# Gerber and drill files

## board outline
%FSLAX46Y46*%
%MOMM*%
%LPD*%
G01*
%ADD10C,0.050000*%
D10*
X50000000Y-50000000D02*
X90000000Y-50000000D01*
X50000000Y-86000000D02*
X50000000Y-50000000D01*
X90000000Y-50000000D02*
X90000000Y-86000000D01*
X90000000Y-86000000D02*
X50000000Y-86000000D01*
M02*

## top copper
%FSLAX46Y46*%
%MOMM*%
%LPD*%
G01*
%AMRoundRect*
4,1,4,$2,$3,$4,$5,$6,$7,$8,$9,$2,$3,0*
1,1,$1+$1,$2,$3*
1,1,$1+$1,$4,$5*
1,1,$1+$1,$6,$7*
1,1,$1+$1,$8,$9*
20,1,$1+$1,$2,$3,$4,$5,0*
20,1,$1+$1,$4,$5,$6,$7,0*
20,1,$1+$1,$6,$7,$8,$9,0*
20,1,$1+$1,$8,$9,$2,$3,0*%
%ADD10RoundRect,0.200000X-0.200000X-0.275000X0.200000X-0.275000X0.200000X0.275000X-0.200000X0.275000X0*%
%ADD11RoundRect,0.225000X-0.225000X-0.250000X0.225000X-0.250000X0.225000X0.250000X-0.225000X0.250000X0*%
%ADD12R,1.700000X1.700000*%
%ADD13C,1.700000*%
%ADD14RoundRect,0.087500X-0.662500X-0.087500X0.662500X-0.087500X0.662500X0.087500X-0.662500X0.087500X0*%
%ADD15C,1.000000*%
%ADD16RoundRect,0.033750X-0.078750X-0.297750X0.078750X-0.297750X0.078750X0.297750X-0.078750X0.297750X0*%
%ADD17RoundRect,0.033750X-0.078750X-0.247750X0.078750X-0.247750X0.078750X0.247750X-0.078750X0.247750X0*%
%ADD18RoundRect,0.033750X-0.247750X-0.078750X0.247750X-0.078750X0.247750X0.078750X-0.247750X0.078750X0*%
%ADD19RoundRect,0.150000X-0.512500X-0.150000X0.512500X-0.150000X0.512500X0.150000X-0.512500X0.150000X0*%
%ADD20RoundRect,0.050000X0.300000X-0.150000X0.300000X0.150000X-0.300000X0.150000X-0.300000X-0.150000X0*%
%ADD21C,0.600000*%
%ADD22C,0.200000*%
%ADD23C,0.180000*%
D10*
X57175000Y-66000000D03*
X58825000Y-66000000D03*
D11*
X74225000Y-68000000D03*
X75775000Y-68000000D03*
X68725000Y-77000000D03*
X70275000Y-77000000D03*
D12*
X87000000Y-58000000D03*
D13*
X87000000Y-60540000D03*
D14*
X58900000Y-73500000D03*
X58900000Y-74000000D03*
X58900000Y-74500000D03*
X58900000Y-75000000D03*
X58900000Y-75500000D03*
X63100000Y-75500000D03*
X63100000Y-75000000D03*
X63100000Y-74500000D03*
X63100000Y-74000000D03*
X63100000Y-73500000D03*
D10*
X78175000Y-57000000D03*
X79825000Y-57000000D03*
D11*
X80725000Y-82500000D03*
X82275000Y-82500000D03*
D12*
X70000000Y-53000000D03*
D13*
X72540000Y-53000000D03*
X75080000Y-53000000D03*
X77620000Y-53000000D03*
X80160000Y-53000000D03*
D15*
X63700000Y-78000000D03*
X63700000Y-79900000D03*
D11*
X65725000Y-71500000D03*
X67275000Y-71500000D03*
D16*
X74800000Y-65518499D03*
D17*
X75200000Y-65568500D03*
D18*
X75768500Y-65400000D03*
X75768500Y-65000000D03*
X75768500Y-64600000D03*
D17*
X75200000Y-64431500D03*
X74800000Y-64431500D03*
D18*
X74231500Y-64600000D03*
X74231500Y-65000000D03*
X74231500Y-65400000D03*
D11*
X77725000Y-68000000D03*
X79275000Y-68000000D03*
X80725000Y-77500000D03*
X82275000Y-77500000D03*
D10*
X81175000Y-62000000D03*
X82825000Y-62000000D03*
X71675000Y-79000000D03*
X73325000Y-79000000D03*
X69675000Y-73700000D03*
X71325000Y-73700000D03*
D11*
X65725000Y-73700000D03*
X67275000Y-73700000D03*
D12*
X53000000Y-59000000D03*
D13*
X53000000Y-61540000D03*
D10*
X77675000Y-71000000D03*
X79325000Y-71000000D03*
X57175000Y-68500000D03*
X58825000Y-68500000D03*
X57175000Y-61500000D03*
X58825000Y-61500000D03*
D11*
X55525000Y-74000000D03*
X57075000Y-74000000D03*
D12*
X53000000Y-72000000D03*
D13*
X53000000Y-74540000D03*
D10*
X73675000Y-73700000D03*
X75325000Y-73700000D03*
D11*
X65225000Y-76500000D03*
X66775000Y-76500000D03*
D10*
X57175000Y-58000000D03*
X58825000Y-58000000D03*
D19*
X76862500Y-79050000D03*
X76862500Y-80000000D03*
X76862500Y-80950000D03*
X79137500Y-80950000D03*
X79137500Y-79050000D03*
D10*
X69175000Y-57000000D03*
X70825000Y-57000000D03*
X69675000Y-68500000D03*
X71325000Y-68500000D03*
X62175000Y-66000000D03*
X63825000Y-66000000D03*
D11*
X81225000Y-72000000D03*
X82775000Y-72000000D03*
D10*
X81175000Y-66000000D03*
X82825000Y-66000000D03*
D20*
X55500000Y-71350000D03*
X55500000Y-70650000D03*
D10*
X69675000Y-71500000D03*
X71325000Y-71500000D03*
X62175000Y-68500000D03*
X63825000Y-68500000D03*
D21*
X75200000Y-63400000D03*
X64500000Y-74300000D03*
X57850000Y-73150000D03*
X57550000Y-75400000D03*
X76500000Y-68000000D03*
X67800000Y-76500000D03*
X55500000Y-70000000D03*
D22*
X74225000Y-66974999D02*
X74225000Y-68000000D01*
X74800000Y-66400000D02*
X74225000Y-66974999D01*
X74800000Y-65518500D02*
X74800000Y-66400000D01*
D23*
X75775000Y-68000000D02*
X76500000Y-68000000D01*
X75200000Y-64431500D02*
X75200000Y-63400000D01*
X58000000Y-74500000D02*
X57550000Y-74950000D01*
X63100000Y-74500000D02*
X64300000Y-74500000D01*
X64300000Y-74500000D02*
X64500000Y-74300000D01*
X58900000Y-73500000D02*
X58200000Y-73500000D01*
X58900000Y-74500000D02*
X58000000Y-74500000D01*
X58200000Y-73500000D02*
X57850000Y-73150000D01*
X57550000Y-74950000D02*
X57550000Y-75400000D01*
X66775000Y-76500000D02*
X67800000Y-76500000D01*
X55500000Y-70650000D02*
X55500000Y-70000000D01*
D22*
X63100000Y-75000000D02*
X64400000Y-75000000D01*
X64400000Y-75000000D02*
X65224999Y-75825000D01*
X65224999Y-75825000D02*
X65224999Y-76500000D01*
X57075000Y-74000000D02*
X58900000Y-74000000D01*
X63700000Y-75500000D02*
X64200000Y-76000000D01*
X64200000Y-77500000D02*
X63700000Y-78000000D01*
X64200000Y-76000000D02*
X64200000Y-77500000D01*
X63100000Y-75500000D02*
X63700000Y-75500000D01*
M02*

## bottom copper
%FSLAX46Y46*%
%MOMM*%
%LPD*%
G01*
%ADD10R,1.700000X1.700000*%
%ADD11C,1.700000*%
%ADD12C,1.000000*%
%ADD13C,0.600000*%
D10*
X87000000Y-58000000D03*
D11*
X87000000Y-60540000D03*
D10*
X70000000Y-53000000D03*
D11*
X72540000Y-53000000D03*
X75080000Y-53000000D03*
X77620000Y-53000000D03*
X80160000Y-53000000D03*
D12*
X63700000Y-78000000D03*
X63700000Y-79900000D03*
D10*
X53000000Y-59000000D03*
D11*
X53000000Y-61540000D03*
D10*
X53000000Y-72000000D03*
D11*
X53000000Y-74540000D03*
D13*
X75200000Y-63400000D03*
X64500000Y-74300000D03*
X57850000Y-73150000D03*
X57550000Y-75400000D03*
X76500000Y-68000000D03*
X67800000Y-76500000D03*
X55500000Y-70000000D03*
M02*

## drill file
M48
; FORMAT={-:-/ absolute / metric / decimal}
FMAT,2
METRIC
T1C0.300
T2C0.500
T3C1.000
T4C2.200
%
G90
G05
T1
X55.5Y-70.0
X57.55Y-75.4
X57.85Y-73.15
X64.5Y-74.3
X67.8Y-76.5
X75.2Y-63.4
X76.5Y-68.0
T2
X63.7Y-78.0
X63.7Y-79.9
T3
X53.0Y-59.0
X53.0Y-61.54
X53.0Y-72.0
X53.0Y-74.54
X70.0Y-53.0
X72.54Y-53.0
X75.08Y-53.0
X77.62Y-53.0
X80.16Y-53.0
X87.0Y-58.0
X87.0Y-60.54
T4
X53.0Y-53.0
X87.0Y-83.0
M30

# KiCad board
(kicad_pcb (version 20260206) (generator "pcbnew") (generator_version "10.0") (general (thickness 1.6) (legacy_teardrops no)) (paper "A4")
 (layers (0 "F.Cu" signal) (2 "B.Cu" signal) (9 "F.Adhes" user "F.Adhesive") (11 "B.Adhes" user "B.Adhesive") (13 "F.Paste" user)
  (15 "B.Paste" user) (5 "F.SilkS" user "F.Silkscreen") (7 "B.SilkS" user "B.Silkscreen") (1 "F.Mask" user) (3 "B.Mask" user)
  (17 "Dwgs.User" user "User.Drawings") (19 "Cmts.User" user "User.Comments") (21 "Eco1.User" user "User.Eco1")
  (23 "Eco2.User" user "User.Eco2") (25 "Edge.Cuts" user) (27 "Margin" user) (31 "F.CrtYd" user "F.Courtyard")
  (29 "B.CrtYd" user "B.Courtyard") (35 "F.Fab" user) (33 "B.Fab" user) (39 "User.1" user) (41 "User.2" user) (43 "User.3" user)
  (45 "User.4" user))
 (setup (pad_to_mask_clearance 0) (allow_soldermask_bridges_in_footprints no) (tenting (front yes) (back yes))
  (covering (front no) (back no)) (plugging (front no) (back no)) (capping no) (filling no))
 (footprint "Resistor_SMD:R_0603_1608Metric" (layer "F.Cu") (at 58 66)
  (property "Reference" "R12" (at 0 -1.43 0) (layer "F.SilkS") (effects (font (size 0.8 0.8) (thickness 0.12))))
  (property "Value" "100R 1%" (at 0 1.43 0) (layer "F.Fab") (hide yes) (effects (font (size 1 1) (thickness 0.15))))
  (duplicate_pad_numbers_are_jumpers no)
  (pad "1" smd roundrect (at -0.825 0) (size 0.8 0.95) (layers "F.Cu" "F.Mask" "F.Paste") (roundrect_rratio 0.25) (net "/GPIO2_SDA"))
  (pad "2" smd roundrect (at 0.825 0) (size 0.8 0.95) (layers "F.Cu" "F.Mask" "F.Paste") (roundrect_rratio 0.25) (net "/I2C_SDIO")))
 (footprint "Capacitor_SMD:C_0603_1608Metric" (layer "F.Cu") (at 75 68)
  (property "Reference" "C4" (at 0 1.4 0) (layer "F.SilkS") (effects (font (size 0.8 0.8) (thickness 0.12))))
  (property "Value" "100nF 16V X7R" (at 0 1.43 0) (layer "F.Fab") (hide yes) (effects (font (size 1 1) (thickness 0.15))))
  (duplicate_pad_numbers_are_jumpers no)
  (pad "1" smd roundrect (at -0.775 0) (size 0.9 0.95) (layers "F.Cu" "F.Mask" "F.Paste") (roundrect_rratio 0.25) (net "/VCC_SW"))
  (pad "2" smd roundrect (at 0.775 0) (size 0.9 0.95) (layers "F.Cu" "F.Mask" "F.Paste") (roundrect_rratio 0.25) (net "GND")))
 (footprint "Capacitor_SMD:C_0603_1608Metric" (layer "F.Cu") (at 69.5 77)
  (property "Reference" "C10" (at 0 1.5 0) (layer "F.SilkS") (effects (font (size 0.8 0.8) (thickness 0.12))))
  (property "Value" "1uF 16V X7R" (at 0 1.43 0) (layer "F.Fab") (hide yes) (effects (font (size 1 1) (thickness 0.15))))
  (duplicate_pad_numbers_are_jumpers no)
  (pad "1" smd roundrect (at -0.775 0) (size 0.9 0.95) (layers "F.Cu" "F.Mask" "F.Paste") (roundrect_rratio 0.25) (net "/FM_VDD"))
  (pad "2" smd roundrect (at 0.775 0) (size 0.9 0.95) (layers "F.Cu" "F.Mask" "F.Paste") (roundrect_rratio 0.25) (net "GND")))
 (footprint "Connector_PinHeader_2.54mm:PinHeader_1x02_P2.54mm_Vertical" (layer "F.Cu") (at 87 58)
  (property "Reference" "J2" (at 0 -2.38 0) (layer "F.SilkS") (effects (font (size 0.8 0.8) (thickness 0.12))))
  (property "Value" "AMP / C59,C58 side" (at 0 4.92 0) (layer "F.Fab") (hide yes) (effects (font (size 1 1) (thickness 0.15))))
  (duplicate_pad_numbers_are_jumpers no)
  (pad "1" thru_hole rect (at 0 0) (size 1.7 1.7) (drill 1) (layers "*.Cu" "*.Mask") (remove_unused_layers no) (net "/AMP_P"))
  (pad "2" thru_hole circle (at 0 2.54) (size 1.7 1.7) (drill 1) (layers "*.Cu" "*.Mask") (remove_unused_layers no) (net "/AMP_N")))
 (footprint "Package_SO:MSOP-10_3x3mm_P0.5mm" (layer "F.Cu") (at 61 74.5)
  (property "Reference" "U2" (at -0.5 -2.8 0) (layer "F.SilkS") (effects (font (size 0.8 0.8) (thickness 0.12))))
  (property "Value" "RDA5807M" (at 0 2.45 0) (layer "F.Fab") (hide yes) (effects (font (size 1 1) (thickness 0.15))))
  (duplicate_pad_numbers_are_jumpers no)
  (pad "1" smd roundrect (at -2.1 -1) (size 1.5 0.35) (layers "F.Cu" "F.Mask" "F.Paste") (roundrect_rratio 0.25) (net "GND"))
  (pad "2" smd roundrect (at -2.1 -0.5) (size 1.5 0.35) (layers "F.Cu" "F.Mask" "F.Paste") (roundrect_rratio 0.25) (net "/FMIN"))
  (pad "3" smd roundrect (at -2.1 0) (size 1.5 0.35) (layers "F.Cu" "F.Mask" "F.Paste") (roundrect_rratio 0.25) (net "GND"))
  (pad "4" smd roundrect (at -2.1 0.5) (size 1.5 0.35) (layers "F.Cu" "F.Mask" "F.Paste") (roundrect_rratio 0.25) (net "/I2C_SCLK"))
  (pad "5" smd roundrect (at -2.1 1) (size 1.5 0.35) (layers "F.Cu" "F.Mask" "F.Paste") (roundrect_rratio 0.25) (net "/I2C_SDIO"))
  (pad "6" smd roundrect (at 2.1 1) (size 1.5 0.35) (layers "F.Cu" "F.Mask" "F.Paste") (roundrect_rratio 0.25) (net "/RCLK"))
  (pad "7" smd roundrect (at 2.1 0.5) (size 1.5 0.35) (layers "F.Cu" "F.Mask" "F.Paste") (roundrect_rratio 0.25) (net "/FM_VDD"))
  (pad "8" smd roundrect (at 2.1 0) (size 1.5 0.35) (layers "F.Cu" "F.Mask" "F.Paste") (roundrect_rratio 0.25) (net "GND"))
  (pad "9" smd roundrect (at 2.1 -0.5) (size 1.5 0.35) (layers "F.Cu" "F.Mask" "F.Paste") (roundrect_rratio 0.25) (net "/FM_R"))
  (pad "10" smd roundrect (at 2.1 -1) (size 1.5 0.35) (layers "F.Cu" "F.Mask" "F.Paste") (roundrect_rratio 0.25) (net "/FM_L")))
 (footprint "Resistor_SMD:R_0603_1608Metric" (layer "F.Cu") (at 79 57)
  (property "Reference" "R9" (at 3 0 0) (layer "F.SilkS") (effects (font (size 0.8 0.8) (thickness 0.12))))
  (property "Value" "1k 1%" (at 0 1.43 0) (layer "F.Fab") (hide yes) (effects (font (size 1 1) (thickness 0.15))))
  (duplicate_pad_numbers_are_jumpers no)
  (pad "1" smd roundrect (at -0.825 0) (size 0.8 0.95) (layers "F.Cu" "F.Mask" "F.Paste") (roundrect_rratio 0.25) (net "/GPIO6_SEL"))
  (pad "2" smd roundrect (at 0.825 0) (size 0.8 0.95) (layers "F.Cu" "F.Mask" "F.Paste") (roundrect_rratio 0.25) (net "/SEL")))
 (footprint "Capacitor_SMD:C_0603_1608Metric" (layer "F.Cu") (at 81.5 82.5)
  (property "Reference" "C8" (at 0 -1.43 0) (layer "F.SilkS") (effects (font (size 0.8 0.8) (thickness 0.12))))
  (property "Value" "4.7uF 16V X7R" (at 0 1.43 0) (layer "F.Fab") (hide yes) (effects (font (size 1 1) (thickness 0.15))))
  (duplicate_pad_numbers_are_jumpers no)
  (pad "1" smd roundrect (at -0.775 0) (size 0.9 0.95) (layers "F.Cu" "F.Mask" "F.Paste") (roundrect_rratio 0.25) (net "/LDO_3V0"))
  (pad "2" smd roundrect (at 0.775 0) (size 0.9 0.95) (layers "F.Cu" "F.Mask" "F.Paste") (roundrect_rratio 0.25) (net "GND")))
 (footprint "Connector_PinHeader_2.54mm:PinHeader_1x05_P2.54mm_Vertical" (layer "F.Cu") (at 70 53 90)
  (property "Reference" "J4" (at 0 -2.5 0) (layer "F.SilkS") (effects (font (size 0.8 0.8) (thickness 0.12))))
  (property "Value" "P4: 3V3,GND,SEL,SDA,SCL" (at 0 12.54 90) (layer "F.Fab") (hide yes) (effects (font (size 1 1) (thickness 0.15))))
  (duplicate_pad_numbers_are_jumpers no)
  (pad "1" thru_hole rect (at 0 0 90) (size 1.7 1.7) (drill 1) (layers "*.Cu" "*.Mask") (remove_unused_layers no) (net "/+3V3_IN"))
  (pad "2" thru_hole circle (at 0 2.54 90) (size 1.7 1.7) (drill 1) (layers "*.Cu" "*.Mask") (remove_unused_layers no) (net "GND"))
  (pad "3" thru_hole circle (at 0 5.08 90) (size 1.7 1.7) (drill 1) (layers "*.Cu" "*.Mask") (remove_unused_layers no) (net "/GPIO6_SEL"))
  (pad "4" thru_hole circle (at 0 7.62 90) (size 1.7 1.7) (drill 1) (layers "*.Cu" "*.Mask") (remove_unused_layers no) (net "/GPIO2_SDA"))
  (pad "5" thru_hole circle (at 0 10.16 90) (size 1.7 1.7) (drill 1) (layers "*.Cu" "*.Mask") (remove_unused_layers no) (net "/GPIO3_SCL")))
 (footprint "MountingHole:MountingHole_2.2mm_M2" (layer "F.Cu") (at 53 53)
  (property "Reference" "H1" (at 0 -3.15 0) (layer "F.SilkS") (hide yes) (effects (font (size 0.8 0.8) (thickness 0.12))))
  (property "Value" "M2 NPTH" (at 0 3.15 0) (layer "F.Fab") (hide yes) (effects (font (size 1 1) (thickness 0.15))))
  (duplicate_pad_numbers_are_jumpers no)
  (pad "" np_thru_hole circle (at 0 0) (size 2.2 2.2) (drill 2.2) (layers "*.Cu" "*.Mask")))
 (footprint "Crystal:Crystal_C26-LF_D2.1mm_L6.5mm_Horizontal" (layer "F.Cu") (at 63.7 78 -90)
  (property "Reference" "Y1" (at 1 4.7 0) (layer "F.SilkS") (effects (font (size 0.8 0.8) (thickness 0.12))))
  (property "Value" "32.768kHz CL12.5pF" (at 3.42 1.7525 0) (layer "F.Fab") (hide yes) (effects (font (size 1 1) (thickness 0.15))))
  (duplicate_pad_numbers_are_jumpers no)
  (pad "1" thru_hole circle (at 0 0 270) (size 1 1) (drill 0.5) (layers "*.Cu" "*.Mask") (remove_unused_layers no) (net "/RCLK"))
  (pad "2" thru_hole circle (at 1.9 0 270) (size 1 1) (drill 0.5) (layers "*.Cu" "*.Mask") (remove_unused_layers no) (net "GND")))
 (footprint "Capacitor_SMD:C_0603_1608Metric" (layer "F.Cu") (at 66.5 71.5)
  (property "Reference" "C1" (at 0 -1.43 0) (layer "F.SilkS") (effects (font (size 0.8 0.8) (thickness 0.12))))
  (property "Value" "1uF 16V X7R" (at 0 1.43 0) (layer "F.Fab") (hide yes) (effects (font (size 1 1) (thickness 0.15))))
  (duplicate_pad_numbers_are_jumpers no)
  (pad "1" smd roundrect (at -0.775 0) (size 0.9 0.95) (layers "F.Cu" "F.Mask" "F.Paste") (roundrect_rratio 0.25) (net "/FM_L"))
  (pad "2" smd roundrect (at 0.775 0) (size 0.9 0.95) (layers "F.Cu" "F.Mask" "F.Paste") (roundrect_rratio 0.25) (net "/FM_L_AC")))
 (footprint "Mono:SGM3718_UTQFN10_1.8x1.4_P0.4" (layer "F.Cu") (at 75 65)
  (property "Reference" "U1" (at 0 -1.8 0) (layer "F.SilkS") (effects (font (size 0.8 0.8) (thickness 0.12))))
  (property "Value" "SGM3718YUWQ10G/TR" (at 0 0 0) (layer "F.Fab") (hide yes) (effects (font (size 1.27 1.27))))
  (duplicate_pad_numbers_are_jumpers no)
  (pad "1" smd roundrect (at -0.2 0.518499) (size 0.225 0.663) (layers "F.Cu" "F.Mask" "F.Paste") (roundrect_rratio 0.15) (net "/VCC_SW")
   (thermal_bridge_angle 45))
  (pad "2" smd roundrect (at 0.2 0.5685) (size 0.225 0.563) (layers "F.Cu" "F.Mask" "F.Paste") (roundrect_rratio 0.15) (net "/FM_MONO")
   (thermal_bridge_angle 45))
  (pad "3" smd roundrect (at 0.7685 0.4) (size 0.563 0.225) (layers "F.Cu" "F.Mask" "F.Paste") (roundrect_rratio 0.15) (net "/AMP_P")
   (thermal_bridge_angle 45))
  (pad "4" smd roundrect (at 0.7685 0) (size 0.563 0.225) (layers "F.Cu" "F.Mask" "F.Paste") (roundrect_rratio 0.15) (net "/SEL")
   (thermal_bridge_angle 45))
  (pad "5" smd roundrect (at 0.7685 -0.4) (size 0.563 0.225) (layers "F.Cu" "F.Mask" "F.Paste") (roundrect_rratio 0.15) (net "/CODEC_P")
   (thermal_bridge_angle 45))
  (pad "6" smd roundrect (at 0.2 -0.5685) (size 0.225 0.563) (layers "F.Cu" "F.Mask" "F.Paste") (roundrect_rratio 0.15) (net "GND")
   (thermal_bridge_angle 45))
  (pad "7" smd roundrect (at -0.2 -0.5685) (size 0.225 0.563) (layers "F.Cu" "F.Mask" "F.Paste") (roundrect_rratio 0.15) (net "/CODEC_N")
   (thermal_bridge_angle 45))
  (pad "8" smd roundrect (at -0.7685 -0.4) (size 0.563 0.225) (layers "F.Cu" "F.Mask" "F.Paste") (roundrect_rratio 0.15) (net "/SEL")
   (thermal_bridge_angle 45))
  (pad "9" smd roundrect (at -0.7685 0) (size 0.563 0.225) (layers "F.Cu" "F.Mask" "F.Paste") (roundrect_rratio 0.15) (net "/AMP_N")
   (thermal_bridge_angle 45))
  (pad "10" smd roundrect (at -0.7685 0.4) (size 0.563 0.225) (layers "F.Cu" "F.Mask" "F.Paste") (roundrect_rratio 0.15) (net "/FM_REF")
   (thermal_bridge_angle 45)))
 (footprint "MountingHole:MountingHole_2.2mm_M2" (layer "F.Cu") (at 87 83)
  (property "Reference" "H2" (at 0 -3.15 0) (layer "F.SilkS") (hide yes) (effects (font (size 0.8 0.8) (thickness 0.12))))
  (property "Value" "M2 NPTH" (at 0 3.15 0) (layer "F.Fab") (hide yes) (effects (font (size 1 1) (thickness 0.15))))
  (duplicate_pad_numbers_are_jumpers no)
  (pad "" np_thru_hole circle (at 0 0) (size 2.2 2.2) (drill 2.2) (layers "*.Cu" "*.Mask")))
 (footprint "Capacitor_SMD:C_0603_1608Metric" (layer "F.Cu") (at 78.5 68)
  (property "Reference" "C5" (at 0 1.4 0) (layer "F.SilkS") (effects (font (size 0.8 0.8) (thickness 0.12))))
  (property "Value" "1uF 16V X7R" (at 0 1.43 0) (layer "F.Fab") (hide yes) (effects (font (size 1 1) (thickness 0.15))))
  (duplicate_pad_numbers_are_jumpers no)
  (pad "1" smd roundrect (at -0.775 0) (size 0.9 0.95) (layers "F.Cu" "F.Mask" "F.Paste") (roundrect_rratio 0.25) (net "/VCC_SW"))
  (pad "2" smd roundrect (at 0.775 0) (size 0.9 0.95) (layers "F.Cu" "F.Mask" "F.Paste") (roundrect_rratio 0.25) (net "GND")))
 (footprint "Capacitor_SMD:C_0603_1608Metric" (layer "F.Cu") (at 81.5 77.5)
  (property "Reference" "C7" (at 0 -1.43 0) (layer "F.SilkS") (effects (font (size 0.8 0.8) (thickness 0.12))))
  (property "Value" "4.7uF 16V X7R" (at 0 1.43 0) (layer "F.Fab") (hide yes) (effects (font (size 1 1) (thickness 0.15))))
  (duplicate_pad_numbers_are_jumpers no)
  (pad "1" smd roundrect (at -0.775 0) (size 0.9 0.95) (layers "F.Cu" "F.Mask" "F.Paste") (roundrect_rratio 0.25) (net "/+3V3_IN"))
  (pad "2" smd roundrect (at 0.775 0) (size 0.9 0.95) (layers "F.Cu" "F.Mask" "F.Paste") (roundrect_rratio 0.25) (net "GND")))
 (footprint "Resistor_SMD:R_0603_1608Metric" (layer "F.Cu") (at 82 62)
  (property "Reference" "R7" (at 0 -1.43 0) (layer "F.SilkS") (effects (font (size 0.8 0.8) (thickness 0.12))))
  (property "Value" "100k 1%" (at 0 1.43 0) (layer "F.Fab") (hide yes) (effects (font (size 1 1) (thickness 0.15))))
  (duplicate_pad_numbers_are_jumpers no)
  (pad "1" smd roundrect (at -0.825 0) (size 0.8 0.95) (layers "F.Cu" "F.Mask" "F.Paste") (roundrect_rratio 0.25) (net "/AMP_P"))
  (pad "2" smd roundrect (at 0.825 0) (size 0.8 0.95) (layers "F.Cu" "F.Mask" "F.Paste") (roundrect_rratio 0.25) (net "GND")))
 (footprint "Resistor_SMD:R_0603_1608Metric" (layer "F.Cu") (at 72.5 79)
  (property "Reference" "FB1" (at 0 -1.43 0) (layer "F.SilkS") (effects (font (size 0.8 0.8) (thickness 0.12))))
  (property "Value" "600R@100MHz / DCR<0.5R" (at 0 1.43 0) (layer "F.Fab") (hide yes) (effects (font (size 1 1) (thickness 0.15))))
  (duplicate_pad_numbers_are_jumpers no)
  (pad "1" smd roundrect (at -0.825 0) (size 0.8 0.95) (layers "F.Cu" "F.Mask" "F.Paste") (roundrect_rratio 0.25) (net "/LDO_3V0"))
  (pad "2" smd roundrect (at 0.825 0) (size 0.8 0.95) (layers "F.Cu" "F.Mask" "F.Paste") (roundrect_rratio 0.25) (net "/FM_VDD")))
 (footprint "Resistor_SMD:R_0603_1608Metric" (layer "F.Cu") (at 70.5 73.7)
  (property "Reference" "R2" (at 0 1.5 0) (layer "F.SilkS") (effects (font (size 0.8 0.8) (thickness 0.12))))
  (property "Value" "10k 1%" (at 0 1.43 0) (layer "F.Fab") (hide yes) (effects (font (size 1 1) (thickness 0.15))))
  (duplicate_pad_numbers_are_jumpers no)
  (pad "1" smd roundrect (at -0.825 0) (size 0.8 0.95) (layers "F.Cu" "F.Mask" "F.Paste") (roundrect_rratio 0.25) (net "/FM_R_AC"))
  (pad "2" smd roundrect (at 0.825 0) (size 0.8 0.95) (layers "F.Cu" "F.Mask" "F.Paste") (roundrect_rratio 0.25) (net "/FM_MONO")))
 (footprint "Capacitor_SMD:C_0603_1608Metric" (layer "F.Cu") (at 66.5 73.7)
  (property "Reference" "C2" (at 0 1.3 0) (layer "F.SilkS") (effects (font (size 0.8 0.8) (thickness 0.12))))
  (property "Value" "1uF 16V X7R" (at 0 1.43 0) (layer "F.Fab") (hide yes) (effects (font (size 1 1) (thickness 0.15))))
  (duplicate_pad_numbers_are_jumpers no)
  (pad "1" smd roundrect (at -0.775 0) (size 0.9 0.95) (layers "F.Cu" "F.Mask" "F.Paste") (roundrect_rratio 0.25) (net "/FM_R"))
  (pad "2" smd roundrect (at 0.775 0) (size 0.9 0.95) (layers "F.Cu" "F.Mask" "F.Paste") (roundrect_rratio 0.25) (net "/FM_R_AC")))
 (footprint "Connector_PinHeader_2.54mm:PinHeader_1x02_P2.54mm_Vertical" (layer "F.Cu") (at 53 59)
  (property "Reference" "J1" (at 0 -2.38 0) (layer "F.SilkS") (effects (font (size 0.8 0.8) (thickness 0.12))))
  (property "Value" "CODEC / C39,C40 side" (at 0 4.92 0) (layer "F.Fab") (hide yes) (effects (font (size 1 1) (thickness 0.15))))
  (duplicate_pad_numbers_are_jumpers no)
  (pad "1" thru_hole rect (at 0 0) (size 1.7 1.7) (drill 1) (layers "*.Cu" "*.Mask") (remove_unused_layers no) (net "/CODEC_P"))
  (pad "2" thru_hole circle (at 0 2.54) (size 1.7 1.7) (drill 1) (layers "*.Cu" "*.Mask") (remove_unused_layers no) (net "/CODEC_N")))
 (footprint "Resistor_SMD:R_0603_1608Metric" (layer "F.Cu") (at 78.5 71)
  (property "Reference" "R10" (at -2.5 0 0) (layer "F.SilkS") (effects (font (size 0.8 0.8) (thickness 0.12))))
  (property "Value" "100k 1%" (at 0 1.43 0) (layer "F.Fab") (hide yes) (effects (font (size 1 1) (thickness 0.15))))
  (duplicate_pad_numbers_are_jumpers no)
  (pad "1" smd roundrect (at -0.825 0) (size 0.8 0.95) (layers "F.Cu" "F.Mask" "F.Paste") (roundrect_rratio 0.25) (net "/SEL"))
  (pad "2" smd roundrect (at 0.825 0) (size 0.8 0.95) (layers "F.Cu" "F.Mask" "F.Paste") (roundrect_rratio 0.25) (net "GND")))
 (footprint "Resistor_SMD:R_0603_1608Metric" (layer "F.Cu") (at 58 68.5)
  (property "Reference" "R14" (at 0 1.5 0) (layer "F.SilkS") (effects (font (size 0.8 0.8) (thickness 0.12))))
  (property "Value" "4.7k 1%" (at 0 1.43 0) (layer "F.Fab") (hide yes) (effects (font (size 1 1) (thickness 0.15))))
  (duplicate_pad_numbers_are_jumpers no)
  (pad "1" smd roundrect (at -0.825 0) (size 0.8 0.95) (layers "F.Cu" "F.Mask" "F.Paste") (roundrect_rratio 0.25) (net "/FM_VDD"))
  (pad "2" smd roundrect (at 0.825 0) (size 0.8 0.95) (layers "F.Cu" "F.Mask" "F.Paste") (roundrect_rratio 0.25) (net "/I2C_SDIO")))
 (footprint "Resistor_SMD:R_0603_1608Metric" (layer "F.Cu") (at 58 61.5)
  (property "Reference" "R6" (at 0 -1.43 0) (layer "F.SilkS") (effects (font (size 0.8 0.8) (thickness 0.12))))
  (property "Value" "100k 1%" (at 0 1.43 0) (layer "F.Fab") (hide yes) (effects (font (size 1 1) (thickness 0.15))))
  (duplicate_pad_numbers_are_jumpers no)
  (pad "1" smd roundrect (at -0.825 0) (size 0.8 0.95) (layers "F.Cu" "F.Mask" "F.Paste") (roundrect_rratio 0.25) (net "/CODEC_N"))
  (pad "2" smd roundrect (at 0.825 0) (size 0.8 0.95) (layers "F.Cu" "F.Mask" "F.Paste") (roundrect_rratio 0.25) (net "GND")))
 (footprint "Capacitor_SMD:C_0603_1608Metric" (layer "F.Cu") (at 56.3 74)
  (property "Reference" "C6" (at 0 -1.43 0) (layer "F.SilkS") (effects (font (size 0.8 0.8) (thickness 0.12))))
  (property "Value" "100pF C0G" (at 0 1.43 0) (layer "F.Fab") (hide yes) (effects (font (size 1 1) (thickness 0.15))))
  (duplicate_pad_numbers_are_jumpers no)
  (pad "1" smd roundrect (at -0.775 0) (size 0.9 0.95) (layers "F.Cu" "F.Mask" "F.Paste") (roundrect_rratio 0.25) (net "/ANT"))
  (pad "2" smd roundrect (at 0.775 0) (size 0.9 0.95) (layers "F.Cu" "F.Mask" "F.Paste") (roundrect_rratio 0.25) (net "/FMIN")))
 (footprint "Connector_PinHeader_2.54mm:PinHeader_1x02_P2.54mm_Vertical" (layer "F.Cu") (at 53 72)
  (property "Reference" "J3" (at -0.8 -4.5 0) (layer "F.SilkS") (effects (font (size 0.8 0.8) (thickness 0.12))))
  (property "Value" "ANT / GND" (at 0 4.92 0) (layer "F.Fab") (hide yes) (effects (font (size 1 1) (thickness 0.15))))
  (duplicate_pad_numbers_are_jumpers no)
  (pad "1" thru_hole rect (at 0 0) (size 1.7 1.7) (drill 1) (layers "*.Cu" "*.Mask") (remove_unused_layers no) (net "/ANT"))
  (pad "2" thru_hole circle (at 0 2.54) (size 1.7 1.7) (drill 1) (layers "*.Cu" "*.Mask") (remove_unused_layers no) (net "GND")))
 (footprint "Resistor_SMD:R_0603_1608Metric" (layer "F.Cu") (at 74.5 73.7)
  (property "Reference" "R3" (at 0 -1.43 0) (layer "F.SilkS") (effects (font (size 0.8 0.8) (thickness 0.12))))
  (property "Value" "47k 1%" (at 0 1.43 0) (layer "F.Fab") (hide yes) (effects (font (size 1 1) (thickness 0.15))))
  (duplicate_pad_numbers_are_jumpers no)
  (pad "1" smd roundrect (at -0.825 0) (size 0.8 0.95) (layers "F.Cu" "F.Mask" "F.Paste") (roundrect_rratio 0.25) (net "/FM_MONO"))
  (pad "2" smd roundrect (at 0.825 0) (size 0.8 0.95) (layers "F.Cu" "F.Mask" "F.Paste") (roundrect_rratio 0.25) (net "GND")))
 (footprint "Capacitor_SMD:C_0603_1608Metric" (layer "F.Cu") (at 66 76.5)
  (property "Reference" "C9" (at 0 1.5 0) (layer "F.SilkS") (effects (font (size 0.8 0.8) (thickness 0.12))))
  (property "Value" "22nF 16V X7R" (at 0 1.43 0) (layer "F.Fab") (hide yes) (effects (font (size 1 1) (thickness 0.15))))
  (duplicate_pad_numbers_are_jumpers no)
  (pad "1" smd roundrect (at -0.775 0) (size 0.9 0.95) (layers "F.Cu" "F.Mask" "F.Paste") (roundrect_rratio 0.25) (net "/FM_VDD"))
  (pad "2" smd roundrect (at 0.775 0) (size 0.9 0.95) (layers "F.Cu" "F.Mask" "F.Paste") (roundrect_rratio 0.25) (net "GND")))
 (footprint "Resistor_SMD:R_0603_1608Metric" (layer "F.Cu") (at 58 58)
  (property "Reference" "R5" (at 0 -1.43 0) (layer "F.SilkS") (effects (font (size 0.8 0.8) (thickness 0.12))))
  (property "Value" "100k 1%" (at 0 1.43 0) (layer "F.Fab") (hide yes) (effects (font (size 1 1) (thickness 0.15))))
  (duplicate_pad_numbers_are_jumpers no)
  (pad "1" smd roundrect (at -0.825 0) (size 0.8 0.95) (layers "F.Cu" "F.Mask" "F.Paste") (roundrect_rratio 0.25) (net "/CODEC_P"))
  (pad "2" smd roundrect (at 0.825 0) (size 0.8 0.95) (layers "F.Cu" "F.Mask" "F.Paste") (roundrect_rratio 0.25) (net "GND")))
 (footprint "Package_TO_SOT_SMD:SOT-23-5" (layer "F.Cu") (at 78 80)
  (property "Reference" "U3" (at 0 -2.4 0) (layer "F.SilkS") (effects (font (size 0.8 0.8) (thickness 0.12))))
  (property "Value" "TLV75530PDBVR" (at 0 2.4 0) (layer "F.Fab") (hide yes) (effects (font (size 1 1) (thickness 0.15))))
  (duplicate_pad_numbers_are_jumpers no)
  (pad "1" smd roundrect (at -1.1375 -0.95) (size 1.325 0.6) (layers "F.Cu" "F.Mask" "F.Paste") (roundrect_rratio 0.25) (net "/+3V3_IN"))
  (pad "2" smd roundrect (at -1.1375 0) (size 1.325 0.6) (layers "F.Cu" "F.Mask" "F.Paste") (roundrect_rratio 0.25) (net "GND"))
  (pad "3" smd roundrect (at -1.1375 0.95) (size 1.325 0.6) (layers "F.Cu" "F.Mask" "F.Paste") (roundrect_rratio 0.25) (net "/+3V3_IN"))
  (pad "4" smd roundrect (at 1.1375 0.95) (size 1.325 0.6) (layers "F.Cu" "F.Mask" "F.Paste") (roundrect_rratio 0.25))
  (pad "5" smd roundrect (at 1.1375 -0.95) (size 1.325 0.6) (layers "F.Cu" "F.Mask" "F.Paste") (roundrect_rratio 0.25) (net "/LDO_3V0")))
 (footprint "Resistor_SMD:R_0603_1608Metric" (layer "F.Cu") (at 70 57)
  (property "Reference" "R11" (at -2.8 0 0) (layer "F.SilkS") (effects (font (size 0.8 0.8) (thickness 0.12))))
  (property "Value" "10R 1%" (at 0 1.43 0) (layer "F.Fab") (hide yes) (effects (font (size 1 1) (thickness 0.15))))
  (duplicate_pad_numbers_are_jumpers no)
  (pad "1" smd roundrect (at -0.825 0) (size 0.8 0.95) (layers "F.Cu" "F.Mask" "F.Paste") (roundrect_rratio 0.25) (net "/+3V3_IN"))
  (pad "2" smd roundrect (at 0.825 0) (size 0.8 0.95) (layers "F.Cu" "F.Mask" "F.Paste") (roundrect_rratio 0.25) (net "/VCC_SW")))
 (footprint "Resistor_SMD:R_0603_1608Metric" (layer "F.Cu") (at 70.5 68.5)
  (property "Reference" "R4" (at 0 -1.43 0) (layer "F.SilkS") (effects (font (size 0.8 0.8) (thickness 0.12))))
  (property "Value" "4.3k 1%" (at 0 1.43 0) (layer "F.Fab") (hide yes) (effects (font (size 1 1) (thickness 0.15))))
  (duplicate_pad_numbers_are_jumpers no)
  (pad "1" smd roundrect (at -0.825 0) (size 0.8 0.95) (layers "F.Cu" "F.Mask" "F.Paste") (roundrect_rratio 0.25) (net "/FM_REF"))
  (pad "2" smd roundrect (at 0.825 0) (size 0.8 0.95) (layers "F.Cu" "F.Mask" "F.Paste") (roundrect_rratio 0.25) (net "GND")))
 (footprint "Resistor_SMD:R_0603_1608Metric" (layer "F.Cu") (at 63 66)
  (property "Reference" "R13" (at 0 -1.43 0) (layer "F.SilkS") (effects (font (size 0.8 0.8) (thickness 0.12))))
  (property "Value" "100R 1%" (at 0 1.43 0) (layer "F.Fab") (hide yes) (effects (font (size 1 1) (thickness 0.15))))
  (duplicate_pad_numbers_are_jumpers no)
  (pad "1" smd roundrect (at -0.825 0) (size 0.8 0.95) (layers "F.Cu" "F.Mask" "F.Paste") (roundrect_rratio 0.25) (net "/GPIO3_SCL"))
  (pad "2" smd roundrect (at 0.825 0) (size 0.8 0.95) (layers "F.Cu" "F.Mask" "F.Paste") (roundrect_rratio 0.25) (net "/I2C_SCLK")))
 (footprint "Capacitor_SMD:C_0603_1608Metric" (layer "F.Cu") (at 82 72)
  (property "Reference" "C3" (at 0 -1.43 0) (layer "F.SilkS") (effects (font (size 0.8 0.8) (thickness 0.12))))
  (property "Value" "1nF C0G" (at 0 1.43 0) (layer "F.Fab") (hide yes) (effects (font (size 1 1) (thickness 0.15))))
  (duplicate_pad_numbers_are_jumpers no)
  (pad "1" smd roundrect (at -0.775 0) (size 0.9 0.95) (layers "F.Cu" "F.Mask" "F.Paste") (roundrect_rratio 0.25) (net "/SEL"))
  (pad "2" smd roundrect (at 0.775 0) (size 0.9 0.95) (layers "F.Cu" "F.Mask" "F.Paste") (roundrect_rratio 0.25) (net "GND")))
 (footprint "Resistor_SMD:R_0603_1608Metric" (layer "F.Cu") (at 82 66)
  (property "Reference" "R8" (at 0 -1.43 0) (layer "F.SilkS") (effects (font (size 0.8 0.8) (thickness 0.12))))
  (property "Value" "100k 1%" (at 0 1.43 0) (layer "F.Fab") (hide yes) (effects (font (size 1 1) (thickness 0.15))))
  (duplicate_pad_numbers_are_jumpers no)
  (pad "1" smd roundrect (at -0.825 0) (size 0.8 0.95) (layers "F.Cu" "F.Mask" "F.Paste") (roundrect_rratio 0.25) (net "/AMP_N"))
  (pad "2" smd roundrect (at 0.825 0) (size 0.8 0.95) (layers "F.Cu" "F.Mask" "F.Paste") (roundrect_rratio 0.25) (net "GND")))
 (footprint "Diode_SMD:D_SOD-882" (layer "F.Cu") (at 55.5 71 90)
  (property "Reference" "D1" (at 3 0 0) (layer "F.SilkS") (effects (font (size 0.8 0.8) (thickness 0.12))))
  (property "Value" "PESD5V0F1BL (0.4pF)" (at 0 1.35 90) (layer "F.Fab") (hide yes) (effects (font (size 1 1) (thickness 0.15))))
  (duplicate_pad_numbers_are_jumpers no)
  (pad "" smd roundrect (at -0.35 0 90) (size 0.3 0.6) (layers "F.Paste") (roundrect_rratio 0.1666666667) (solder_paste_margin -0.05))
  (pad "" smd roundrect (at 0.35 0 90) (size 0.3 0.6) (layers "F.Paste") (roundrect_rratio 0.1666666667) (solder_paste_margin -0.05))
  (pad "1" smd roundrect (at -0.35 0 90) (size 0.4 0.7) (layers "F.Cu" "F.Mask") (roundrect_rratio 0.125) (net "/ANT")
   (solder_paste_margin -0.05))
  (pad "2" smd roundrect (at 0.35 0 90) (size 0.4 0.7) (layers "F.Cu" "F.Mask") (roundrect_rratio 0.125) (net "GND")
   (solder_paste_margin -0.05)))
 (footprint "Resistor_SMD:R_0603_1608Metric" (layer "F.Cu") (at 70.5 71.5)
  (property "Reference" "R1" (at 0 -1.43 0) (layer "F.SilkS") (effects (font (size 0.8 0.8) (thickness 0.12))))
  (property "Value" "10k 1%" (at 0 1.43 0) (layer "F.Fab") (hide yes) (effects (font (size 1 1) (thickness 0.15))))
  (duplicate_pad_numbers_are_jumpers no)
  (pad "1" smd roundrect (at -0.825 0) (size 0.8 0.95) (layers "F.Cu" "F.Mask" "F.Paste") (roundrect_rratio 0.25) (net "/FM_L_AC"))
  (pad "2" smd roundrect (at 0.825 0) (size 0.8 0.95) (layers "F.Cu" "F.Mask" "F.Paste") (roundrect_rratio 0.25) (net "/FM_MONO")))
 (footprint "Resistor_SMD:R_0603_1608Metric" (layer "F.Cu") (at 63 68.5)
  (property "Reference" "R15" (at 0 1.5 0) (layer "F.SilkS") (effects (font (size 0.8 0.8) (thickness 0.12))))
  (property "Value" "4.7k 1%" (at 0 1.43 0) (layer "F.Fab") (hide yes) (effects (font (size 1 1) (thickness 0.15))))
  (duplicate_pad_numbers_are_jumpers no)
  (pad "1" smd roundrect (at -0.825 0) (size 0.8 0.95) (layers "F.Cu" "F.Mask" "F.Paste") (roundrect_rratio 0.25) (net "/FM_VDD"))
  (pad "2" smd roundrect (at 0.825 0) (size 0.8 0.95) (layers "F.Cu" "F.Mask" "F.Paste") (roundrect_rratio 0.25) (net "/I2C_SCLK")))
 (gr_line (start 50 50) (end 90 50) (stroke (width 0.05) (type default)) (layer "Edge.Cuts"))
 (gr_line (start 50 86) (end 50 50) (stroke (width 0.05) (type default)) (layer "Edge.Cuts"))
 (gr_line (start 90 50) (end 90 86) (stroke (width 0.05) (type default)) (layer "Edge.Cuts"))
 (gr_line (start 90 86) (end 50 86) (stroke (width 0.05) (type default)) (layer "Edge.Cuts"))
 (segment (start 74.225 66.974999) (end 74.225 68) (width 0.2) (locked yes) (layer "F.Cu") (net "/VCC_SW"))
 (segment (start 74.8 66.4) (end 74.225 66.974999) (width 0.2) (locked yes) (layer "F.Cu") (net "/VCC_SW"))
 (segment (start 74.8 65.5185) (end 74.8 66.4) (width 0.2) (locked yes) (layer "F.Cu") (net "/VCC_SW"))
 (segment (start 75.775 68) (end 76.5 68) (width 0.18) (locked yes) (layer "F.Cu") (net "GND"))
 (segment (start 75.2 64.4315) (end 75.2 63.4) (width 0.18) (locked yes) (layer "F.Cu") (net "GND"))
 (segment (start 58 74.5) (end 57.55 74.95) (width 0.18) (locked yes) (layer "F.Cu") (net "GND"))
 (segment (start 63.1 74.5) (end 64.3 74.5) (width 0.18) (locked yes) (layer "F.Cu") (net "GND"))
 (segment (start 64.3 74.5) (end 64.5 74.3) (width 0.18) (locked yes) (layer "F.Cu") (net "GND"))
 (segment (start 58.9 73.5) (end 58.2 73.5) (width 0.18) (locked yes) (layer "F.Cu") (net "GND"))
 (segment (start 58.9 74.5) (end 58 74.5) (width 0.18) (locked yes) (layer "F.Cu") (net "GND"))
 (segment (start 58.2 73.5) (end 57.85 73.15) (width 0.18) (locked yes) (layer "F.Cu") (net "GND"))
 (segment (start 57.55 74.95) (end 57.55 75.4) (width 0.18) (locked yes) (layer "F.Cu") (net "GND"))
 (segment (start 66.775 76.5) (end 67.8 76.5) (width 0.18) (locked yes) (layer "F.Cu") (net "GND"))
 (segment (start 55.5 70.65) (end 55.5 70) (width 0.18) (locked yes) (layer "F.Cu") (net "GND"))
 (via (at 75.2 63.4) (size 0.6) (drill 0.3) (layers "F.Cu" "B.Cu") (locked yes) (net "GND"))
 (via (at 64.5 74.3) (size 0.6) (drill 0.3) (layers "F.Cu" "B.Cu") (locked yes) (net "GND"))
 (via (at 57.85 73.15) (size 0.6) (drill 0.3) (layers "F.Cu" "B.Cu") (locked yes) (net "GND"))
 (via (at 57.55 75.4) (size 0.6) (drill 0.3) (layers "F.Cu" "B.Cu") (locked yes) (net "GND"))
 (via (at 76.5 68) (size 0.6) (drill 0.3) (layers "F.Cu" "B.Cu") (locked yes) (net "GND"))
 (via (at 67.8 76.5) (size 0.6) (drill 0.3) (layers "F.Cu" "B.Cu") (locked yes) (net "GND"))
 (via (at 55.5 70) (size 0.6) (drill 0.3) (layers "F.Cu" "B.Cu") (locked yes) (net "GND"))
 (segment (start 63.1 75) (end 64.4 75) (width 0.2) (locked yes) (layer "F.Cu") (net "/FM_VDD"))
 (segment (start 64.4 75) (end 65.224999 75.825) (width 0.2) (locked yes) (layer "F.Cu") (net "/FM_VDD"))
 (segment (start 65.224999 75.825) (end 65.224999 76.5) (width 0.2) (locked yes) (layer "F.Cu") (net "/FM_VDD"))
 (segment (start 57.075 74) (end 58.9 74) (width 0.2) (locked yes) (layer "F.Cu") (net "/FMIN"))
 (segment (start 63.7 75.5) (end 64.2 76) (width 0.2) (locked yes) (layer "F.Cu") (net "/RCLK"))
 (segment (start 64.2 77.5) (end 63.7 78) (width 0.2) (locked yes) (layer "F.Cu") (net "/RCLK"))
 (segment (start 64.2 76) (end 64.2 77.5) (width 0.2) (locked yes) (layer "F.Cu") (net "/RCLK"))
 (segment (start 63.1 75.5) (end 63.7 75.5) (width 0.2) (locked yes) (layer "F.Cu") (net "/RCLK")))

